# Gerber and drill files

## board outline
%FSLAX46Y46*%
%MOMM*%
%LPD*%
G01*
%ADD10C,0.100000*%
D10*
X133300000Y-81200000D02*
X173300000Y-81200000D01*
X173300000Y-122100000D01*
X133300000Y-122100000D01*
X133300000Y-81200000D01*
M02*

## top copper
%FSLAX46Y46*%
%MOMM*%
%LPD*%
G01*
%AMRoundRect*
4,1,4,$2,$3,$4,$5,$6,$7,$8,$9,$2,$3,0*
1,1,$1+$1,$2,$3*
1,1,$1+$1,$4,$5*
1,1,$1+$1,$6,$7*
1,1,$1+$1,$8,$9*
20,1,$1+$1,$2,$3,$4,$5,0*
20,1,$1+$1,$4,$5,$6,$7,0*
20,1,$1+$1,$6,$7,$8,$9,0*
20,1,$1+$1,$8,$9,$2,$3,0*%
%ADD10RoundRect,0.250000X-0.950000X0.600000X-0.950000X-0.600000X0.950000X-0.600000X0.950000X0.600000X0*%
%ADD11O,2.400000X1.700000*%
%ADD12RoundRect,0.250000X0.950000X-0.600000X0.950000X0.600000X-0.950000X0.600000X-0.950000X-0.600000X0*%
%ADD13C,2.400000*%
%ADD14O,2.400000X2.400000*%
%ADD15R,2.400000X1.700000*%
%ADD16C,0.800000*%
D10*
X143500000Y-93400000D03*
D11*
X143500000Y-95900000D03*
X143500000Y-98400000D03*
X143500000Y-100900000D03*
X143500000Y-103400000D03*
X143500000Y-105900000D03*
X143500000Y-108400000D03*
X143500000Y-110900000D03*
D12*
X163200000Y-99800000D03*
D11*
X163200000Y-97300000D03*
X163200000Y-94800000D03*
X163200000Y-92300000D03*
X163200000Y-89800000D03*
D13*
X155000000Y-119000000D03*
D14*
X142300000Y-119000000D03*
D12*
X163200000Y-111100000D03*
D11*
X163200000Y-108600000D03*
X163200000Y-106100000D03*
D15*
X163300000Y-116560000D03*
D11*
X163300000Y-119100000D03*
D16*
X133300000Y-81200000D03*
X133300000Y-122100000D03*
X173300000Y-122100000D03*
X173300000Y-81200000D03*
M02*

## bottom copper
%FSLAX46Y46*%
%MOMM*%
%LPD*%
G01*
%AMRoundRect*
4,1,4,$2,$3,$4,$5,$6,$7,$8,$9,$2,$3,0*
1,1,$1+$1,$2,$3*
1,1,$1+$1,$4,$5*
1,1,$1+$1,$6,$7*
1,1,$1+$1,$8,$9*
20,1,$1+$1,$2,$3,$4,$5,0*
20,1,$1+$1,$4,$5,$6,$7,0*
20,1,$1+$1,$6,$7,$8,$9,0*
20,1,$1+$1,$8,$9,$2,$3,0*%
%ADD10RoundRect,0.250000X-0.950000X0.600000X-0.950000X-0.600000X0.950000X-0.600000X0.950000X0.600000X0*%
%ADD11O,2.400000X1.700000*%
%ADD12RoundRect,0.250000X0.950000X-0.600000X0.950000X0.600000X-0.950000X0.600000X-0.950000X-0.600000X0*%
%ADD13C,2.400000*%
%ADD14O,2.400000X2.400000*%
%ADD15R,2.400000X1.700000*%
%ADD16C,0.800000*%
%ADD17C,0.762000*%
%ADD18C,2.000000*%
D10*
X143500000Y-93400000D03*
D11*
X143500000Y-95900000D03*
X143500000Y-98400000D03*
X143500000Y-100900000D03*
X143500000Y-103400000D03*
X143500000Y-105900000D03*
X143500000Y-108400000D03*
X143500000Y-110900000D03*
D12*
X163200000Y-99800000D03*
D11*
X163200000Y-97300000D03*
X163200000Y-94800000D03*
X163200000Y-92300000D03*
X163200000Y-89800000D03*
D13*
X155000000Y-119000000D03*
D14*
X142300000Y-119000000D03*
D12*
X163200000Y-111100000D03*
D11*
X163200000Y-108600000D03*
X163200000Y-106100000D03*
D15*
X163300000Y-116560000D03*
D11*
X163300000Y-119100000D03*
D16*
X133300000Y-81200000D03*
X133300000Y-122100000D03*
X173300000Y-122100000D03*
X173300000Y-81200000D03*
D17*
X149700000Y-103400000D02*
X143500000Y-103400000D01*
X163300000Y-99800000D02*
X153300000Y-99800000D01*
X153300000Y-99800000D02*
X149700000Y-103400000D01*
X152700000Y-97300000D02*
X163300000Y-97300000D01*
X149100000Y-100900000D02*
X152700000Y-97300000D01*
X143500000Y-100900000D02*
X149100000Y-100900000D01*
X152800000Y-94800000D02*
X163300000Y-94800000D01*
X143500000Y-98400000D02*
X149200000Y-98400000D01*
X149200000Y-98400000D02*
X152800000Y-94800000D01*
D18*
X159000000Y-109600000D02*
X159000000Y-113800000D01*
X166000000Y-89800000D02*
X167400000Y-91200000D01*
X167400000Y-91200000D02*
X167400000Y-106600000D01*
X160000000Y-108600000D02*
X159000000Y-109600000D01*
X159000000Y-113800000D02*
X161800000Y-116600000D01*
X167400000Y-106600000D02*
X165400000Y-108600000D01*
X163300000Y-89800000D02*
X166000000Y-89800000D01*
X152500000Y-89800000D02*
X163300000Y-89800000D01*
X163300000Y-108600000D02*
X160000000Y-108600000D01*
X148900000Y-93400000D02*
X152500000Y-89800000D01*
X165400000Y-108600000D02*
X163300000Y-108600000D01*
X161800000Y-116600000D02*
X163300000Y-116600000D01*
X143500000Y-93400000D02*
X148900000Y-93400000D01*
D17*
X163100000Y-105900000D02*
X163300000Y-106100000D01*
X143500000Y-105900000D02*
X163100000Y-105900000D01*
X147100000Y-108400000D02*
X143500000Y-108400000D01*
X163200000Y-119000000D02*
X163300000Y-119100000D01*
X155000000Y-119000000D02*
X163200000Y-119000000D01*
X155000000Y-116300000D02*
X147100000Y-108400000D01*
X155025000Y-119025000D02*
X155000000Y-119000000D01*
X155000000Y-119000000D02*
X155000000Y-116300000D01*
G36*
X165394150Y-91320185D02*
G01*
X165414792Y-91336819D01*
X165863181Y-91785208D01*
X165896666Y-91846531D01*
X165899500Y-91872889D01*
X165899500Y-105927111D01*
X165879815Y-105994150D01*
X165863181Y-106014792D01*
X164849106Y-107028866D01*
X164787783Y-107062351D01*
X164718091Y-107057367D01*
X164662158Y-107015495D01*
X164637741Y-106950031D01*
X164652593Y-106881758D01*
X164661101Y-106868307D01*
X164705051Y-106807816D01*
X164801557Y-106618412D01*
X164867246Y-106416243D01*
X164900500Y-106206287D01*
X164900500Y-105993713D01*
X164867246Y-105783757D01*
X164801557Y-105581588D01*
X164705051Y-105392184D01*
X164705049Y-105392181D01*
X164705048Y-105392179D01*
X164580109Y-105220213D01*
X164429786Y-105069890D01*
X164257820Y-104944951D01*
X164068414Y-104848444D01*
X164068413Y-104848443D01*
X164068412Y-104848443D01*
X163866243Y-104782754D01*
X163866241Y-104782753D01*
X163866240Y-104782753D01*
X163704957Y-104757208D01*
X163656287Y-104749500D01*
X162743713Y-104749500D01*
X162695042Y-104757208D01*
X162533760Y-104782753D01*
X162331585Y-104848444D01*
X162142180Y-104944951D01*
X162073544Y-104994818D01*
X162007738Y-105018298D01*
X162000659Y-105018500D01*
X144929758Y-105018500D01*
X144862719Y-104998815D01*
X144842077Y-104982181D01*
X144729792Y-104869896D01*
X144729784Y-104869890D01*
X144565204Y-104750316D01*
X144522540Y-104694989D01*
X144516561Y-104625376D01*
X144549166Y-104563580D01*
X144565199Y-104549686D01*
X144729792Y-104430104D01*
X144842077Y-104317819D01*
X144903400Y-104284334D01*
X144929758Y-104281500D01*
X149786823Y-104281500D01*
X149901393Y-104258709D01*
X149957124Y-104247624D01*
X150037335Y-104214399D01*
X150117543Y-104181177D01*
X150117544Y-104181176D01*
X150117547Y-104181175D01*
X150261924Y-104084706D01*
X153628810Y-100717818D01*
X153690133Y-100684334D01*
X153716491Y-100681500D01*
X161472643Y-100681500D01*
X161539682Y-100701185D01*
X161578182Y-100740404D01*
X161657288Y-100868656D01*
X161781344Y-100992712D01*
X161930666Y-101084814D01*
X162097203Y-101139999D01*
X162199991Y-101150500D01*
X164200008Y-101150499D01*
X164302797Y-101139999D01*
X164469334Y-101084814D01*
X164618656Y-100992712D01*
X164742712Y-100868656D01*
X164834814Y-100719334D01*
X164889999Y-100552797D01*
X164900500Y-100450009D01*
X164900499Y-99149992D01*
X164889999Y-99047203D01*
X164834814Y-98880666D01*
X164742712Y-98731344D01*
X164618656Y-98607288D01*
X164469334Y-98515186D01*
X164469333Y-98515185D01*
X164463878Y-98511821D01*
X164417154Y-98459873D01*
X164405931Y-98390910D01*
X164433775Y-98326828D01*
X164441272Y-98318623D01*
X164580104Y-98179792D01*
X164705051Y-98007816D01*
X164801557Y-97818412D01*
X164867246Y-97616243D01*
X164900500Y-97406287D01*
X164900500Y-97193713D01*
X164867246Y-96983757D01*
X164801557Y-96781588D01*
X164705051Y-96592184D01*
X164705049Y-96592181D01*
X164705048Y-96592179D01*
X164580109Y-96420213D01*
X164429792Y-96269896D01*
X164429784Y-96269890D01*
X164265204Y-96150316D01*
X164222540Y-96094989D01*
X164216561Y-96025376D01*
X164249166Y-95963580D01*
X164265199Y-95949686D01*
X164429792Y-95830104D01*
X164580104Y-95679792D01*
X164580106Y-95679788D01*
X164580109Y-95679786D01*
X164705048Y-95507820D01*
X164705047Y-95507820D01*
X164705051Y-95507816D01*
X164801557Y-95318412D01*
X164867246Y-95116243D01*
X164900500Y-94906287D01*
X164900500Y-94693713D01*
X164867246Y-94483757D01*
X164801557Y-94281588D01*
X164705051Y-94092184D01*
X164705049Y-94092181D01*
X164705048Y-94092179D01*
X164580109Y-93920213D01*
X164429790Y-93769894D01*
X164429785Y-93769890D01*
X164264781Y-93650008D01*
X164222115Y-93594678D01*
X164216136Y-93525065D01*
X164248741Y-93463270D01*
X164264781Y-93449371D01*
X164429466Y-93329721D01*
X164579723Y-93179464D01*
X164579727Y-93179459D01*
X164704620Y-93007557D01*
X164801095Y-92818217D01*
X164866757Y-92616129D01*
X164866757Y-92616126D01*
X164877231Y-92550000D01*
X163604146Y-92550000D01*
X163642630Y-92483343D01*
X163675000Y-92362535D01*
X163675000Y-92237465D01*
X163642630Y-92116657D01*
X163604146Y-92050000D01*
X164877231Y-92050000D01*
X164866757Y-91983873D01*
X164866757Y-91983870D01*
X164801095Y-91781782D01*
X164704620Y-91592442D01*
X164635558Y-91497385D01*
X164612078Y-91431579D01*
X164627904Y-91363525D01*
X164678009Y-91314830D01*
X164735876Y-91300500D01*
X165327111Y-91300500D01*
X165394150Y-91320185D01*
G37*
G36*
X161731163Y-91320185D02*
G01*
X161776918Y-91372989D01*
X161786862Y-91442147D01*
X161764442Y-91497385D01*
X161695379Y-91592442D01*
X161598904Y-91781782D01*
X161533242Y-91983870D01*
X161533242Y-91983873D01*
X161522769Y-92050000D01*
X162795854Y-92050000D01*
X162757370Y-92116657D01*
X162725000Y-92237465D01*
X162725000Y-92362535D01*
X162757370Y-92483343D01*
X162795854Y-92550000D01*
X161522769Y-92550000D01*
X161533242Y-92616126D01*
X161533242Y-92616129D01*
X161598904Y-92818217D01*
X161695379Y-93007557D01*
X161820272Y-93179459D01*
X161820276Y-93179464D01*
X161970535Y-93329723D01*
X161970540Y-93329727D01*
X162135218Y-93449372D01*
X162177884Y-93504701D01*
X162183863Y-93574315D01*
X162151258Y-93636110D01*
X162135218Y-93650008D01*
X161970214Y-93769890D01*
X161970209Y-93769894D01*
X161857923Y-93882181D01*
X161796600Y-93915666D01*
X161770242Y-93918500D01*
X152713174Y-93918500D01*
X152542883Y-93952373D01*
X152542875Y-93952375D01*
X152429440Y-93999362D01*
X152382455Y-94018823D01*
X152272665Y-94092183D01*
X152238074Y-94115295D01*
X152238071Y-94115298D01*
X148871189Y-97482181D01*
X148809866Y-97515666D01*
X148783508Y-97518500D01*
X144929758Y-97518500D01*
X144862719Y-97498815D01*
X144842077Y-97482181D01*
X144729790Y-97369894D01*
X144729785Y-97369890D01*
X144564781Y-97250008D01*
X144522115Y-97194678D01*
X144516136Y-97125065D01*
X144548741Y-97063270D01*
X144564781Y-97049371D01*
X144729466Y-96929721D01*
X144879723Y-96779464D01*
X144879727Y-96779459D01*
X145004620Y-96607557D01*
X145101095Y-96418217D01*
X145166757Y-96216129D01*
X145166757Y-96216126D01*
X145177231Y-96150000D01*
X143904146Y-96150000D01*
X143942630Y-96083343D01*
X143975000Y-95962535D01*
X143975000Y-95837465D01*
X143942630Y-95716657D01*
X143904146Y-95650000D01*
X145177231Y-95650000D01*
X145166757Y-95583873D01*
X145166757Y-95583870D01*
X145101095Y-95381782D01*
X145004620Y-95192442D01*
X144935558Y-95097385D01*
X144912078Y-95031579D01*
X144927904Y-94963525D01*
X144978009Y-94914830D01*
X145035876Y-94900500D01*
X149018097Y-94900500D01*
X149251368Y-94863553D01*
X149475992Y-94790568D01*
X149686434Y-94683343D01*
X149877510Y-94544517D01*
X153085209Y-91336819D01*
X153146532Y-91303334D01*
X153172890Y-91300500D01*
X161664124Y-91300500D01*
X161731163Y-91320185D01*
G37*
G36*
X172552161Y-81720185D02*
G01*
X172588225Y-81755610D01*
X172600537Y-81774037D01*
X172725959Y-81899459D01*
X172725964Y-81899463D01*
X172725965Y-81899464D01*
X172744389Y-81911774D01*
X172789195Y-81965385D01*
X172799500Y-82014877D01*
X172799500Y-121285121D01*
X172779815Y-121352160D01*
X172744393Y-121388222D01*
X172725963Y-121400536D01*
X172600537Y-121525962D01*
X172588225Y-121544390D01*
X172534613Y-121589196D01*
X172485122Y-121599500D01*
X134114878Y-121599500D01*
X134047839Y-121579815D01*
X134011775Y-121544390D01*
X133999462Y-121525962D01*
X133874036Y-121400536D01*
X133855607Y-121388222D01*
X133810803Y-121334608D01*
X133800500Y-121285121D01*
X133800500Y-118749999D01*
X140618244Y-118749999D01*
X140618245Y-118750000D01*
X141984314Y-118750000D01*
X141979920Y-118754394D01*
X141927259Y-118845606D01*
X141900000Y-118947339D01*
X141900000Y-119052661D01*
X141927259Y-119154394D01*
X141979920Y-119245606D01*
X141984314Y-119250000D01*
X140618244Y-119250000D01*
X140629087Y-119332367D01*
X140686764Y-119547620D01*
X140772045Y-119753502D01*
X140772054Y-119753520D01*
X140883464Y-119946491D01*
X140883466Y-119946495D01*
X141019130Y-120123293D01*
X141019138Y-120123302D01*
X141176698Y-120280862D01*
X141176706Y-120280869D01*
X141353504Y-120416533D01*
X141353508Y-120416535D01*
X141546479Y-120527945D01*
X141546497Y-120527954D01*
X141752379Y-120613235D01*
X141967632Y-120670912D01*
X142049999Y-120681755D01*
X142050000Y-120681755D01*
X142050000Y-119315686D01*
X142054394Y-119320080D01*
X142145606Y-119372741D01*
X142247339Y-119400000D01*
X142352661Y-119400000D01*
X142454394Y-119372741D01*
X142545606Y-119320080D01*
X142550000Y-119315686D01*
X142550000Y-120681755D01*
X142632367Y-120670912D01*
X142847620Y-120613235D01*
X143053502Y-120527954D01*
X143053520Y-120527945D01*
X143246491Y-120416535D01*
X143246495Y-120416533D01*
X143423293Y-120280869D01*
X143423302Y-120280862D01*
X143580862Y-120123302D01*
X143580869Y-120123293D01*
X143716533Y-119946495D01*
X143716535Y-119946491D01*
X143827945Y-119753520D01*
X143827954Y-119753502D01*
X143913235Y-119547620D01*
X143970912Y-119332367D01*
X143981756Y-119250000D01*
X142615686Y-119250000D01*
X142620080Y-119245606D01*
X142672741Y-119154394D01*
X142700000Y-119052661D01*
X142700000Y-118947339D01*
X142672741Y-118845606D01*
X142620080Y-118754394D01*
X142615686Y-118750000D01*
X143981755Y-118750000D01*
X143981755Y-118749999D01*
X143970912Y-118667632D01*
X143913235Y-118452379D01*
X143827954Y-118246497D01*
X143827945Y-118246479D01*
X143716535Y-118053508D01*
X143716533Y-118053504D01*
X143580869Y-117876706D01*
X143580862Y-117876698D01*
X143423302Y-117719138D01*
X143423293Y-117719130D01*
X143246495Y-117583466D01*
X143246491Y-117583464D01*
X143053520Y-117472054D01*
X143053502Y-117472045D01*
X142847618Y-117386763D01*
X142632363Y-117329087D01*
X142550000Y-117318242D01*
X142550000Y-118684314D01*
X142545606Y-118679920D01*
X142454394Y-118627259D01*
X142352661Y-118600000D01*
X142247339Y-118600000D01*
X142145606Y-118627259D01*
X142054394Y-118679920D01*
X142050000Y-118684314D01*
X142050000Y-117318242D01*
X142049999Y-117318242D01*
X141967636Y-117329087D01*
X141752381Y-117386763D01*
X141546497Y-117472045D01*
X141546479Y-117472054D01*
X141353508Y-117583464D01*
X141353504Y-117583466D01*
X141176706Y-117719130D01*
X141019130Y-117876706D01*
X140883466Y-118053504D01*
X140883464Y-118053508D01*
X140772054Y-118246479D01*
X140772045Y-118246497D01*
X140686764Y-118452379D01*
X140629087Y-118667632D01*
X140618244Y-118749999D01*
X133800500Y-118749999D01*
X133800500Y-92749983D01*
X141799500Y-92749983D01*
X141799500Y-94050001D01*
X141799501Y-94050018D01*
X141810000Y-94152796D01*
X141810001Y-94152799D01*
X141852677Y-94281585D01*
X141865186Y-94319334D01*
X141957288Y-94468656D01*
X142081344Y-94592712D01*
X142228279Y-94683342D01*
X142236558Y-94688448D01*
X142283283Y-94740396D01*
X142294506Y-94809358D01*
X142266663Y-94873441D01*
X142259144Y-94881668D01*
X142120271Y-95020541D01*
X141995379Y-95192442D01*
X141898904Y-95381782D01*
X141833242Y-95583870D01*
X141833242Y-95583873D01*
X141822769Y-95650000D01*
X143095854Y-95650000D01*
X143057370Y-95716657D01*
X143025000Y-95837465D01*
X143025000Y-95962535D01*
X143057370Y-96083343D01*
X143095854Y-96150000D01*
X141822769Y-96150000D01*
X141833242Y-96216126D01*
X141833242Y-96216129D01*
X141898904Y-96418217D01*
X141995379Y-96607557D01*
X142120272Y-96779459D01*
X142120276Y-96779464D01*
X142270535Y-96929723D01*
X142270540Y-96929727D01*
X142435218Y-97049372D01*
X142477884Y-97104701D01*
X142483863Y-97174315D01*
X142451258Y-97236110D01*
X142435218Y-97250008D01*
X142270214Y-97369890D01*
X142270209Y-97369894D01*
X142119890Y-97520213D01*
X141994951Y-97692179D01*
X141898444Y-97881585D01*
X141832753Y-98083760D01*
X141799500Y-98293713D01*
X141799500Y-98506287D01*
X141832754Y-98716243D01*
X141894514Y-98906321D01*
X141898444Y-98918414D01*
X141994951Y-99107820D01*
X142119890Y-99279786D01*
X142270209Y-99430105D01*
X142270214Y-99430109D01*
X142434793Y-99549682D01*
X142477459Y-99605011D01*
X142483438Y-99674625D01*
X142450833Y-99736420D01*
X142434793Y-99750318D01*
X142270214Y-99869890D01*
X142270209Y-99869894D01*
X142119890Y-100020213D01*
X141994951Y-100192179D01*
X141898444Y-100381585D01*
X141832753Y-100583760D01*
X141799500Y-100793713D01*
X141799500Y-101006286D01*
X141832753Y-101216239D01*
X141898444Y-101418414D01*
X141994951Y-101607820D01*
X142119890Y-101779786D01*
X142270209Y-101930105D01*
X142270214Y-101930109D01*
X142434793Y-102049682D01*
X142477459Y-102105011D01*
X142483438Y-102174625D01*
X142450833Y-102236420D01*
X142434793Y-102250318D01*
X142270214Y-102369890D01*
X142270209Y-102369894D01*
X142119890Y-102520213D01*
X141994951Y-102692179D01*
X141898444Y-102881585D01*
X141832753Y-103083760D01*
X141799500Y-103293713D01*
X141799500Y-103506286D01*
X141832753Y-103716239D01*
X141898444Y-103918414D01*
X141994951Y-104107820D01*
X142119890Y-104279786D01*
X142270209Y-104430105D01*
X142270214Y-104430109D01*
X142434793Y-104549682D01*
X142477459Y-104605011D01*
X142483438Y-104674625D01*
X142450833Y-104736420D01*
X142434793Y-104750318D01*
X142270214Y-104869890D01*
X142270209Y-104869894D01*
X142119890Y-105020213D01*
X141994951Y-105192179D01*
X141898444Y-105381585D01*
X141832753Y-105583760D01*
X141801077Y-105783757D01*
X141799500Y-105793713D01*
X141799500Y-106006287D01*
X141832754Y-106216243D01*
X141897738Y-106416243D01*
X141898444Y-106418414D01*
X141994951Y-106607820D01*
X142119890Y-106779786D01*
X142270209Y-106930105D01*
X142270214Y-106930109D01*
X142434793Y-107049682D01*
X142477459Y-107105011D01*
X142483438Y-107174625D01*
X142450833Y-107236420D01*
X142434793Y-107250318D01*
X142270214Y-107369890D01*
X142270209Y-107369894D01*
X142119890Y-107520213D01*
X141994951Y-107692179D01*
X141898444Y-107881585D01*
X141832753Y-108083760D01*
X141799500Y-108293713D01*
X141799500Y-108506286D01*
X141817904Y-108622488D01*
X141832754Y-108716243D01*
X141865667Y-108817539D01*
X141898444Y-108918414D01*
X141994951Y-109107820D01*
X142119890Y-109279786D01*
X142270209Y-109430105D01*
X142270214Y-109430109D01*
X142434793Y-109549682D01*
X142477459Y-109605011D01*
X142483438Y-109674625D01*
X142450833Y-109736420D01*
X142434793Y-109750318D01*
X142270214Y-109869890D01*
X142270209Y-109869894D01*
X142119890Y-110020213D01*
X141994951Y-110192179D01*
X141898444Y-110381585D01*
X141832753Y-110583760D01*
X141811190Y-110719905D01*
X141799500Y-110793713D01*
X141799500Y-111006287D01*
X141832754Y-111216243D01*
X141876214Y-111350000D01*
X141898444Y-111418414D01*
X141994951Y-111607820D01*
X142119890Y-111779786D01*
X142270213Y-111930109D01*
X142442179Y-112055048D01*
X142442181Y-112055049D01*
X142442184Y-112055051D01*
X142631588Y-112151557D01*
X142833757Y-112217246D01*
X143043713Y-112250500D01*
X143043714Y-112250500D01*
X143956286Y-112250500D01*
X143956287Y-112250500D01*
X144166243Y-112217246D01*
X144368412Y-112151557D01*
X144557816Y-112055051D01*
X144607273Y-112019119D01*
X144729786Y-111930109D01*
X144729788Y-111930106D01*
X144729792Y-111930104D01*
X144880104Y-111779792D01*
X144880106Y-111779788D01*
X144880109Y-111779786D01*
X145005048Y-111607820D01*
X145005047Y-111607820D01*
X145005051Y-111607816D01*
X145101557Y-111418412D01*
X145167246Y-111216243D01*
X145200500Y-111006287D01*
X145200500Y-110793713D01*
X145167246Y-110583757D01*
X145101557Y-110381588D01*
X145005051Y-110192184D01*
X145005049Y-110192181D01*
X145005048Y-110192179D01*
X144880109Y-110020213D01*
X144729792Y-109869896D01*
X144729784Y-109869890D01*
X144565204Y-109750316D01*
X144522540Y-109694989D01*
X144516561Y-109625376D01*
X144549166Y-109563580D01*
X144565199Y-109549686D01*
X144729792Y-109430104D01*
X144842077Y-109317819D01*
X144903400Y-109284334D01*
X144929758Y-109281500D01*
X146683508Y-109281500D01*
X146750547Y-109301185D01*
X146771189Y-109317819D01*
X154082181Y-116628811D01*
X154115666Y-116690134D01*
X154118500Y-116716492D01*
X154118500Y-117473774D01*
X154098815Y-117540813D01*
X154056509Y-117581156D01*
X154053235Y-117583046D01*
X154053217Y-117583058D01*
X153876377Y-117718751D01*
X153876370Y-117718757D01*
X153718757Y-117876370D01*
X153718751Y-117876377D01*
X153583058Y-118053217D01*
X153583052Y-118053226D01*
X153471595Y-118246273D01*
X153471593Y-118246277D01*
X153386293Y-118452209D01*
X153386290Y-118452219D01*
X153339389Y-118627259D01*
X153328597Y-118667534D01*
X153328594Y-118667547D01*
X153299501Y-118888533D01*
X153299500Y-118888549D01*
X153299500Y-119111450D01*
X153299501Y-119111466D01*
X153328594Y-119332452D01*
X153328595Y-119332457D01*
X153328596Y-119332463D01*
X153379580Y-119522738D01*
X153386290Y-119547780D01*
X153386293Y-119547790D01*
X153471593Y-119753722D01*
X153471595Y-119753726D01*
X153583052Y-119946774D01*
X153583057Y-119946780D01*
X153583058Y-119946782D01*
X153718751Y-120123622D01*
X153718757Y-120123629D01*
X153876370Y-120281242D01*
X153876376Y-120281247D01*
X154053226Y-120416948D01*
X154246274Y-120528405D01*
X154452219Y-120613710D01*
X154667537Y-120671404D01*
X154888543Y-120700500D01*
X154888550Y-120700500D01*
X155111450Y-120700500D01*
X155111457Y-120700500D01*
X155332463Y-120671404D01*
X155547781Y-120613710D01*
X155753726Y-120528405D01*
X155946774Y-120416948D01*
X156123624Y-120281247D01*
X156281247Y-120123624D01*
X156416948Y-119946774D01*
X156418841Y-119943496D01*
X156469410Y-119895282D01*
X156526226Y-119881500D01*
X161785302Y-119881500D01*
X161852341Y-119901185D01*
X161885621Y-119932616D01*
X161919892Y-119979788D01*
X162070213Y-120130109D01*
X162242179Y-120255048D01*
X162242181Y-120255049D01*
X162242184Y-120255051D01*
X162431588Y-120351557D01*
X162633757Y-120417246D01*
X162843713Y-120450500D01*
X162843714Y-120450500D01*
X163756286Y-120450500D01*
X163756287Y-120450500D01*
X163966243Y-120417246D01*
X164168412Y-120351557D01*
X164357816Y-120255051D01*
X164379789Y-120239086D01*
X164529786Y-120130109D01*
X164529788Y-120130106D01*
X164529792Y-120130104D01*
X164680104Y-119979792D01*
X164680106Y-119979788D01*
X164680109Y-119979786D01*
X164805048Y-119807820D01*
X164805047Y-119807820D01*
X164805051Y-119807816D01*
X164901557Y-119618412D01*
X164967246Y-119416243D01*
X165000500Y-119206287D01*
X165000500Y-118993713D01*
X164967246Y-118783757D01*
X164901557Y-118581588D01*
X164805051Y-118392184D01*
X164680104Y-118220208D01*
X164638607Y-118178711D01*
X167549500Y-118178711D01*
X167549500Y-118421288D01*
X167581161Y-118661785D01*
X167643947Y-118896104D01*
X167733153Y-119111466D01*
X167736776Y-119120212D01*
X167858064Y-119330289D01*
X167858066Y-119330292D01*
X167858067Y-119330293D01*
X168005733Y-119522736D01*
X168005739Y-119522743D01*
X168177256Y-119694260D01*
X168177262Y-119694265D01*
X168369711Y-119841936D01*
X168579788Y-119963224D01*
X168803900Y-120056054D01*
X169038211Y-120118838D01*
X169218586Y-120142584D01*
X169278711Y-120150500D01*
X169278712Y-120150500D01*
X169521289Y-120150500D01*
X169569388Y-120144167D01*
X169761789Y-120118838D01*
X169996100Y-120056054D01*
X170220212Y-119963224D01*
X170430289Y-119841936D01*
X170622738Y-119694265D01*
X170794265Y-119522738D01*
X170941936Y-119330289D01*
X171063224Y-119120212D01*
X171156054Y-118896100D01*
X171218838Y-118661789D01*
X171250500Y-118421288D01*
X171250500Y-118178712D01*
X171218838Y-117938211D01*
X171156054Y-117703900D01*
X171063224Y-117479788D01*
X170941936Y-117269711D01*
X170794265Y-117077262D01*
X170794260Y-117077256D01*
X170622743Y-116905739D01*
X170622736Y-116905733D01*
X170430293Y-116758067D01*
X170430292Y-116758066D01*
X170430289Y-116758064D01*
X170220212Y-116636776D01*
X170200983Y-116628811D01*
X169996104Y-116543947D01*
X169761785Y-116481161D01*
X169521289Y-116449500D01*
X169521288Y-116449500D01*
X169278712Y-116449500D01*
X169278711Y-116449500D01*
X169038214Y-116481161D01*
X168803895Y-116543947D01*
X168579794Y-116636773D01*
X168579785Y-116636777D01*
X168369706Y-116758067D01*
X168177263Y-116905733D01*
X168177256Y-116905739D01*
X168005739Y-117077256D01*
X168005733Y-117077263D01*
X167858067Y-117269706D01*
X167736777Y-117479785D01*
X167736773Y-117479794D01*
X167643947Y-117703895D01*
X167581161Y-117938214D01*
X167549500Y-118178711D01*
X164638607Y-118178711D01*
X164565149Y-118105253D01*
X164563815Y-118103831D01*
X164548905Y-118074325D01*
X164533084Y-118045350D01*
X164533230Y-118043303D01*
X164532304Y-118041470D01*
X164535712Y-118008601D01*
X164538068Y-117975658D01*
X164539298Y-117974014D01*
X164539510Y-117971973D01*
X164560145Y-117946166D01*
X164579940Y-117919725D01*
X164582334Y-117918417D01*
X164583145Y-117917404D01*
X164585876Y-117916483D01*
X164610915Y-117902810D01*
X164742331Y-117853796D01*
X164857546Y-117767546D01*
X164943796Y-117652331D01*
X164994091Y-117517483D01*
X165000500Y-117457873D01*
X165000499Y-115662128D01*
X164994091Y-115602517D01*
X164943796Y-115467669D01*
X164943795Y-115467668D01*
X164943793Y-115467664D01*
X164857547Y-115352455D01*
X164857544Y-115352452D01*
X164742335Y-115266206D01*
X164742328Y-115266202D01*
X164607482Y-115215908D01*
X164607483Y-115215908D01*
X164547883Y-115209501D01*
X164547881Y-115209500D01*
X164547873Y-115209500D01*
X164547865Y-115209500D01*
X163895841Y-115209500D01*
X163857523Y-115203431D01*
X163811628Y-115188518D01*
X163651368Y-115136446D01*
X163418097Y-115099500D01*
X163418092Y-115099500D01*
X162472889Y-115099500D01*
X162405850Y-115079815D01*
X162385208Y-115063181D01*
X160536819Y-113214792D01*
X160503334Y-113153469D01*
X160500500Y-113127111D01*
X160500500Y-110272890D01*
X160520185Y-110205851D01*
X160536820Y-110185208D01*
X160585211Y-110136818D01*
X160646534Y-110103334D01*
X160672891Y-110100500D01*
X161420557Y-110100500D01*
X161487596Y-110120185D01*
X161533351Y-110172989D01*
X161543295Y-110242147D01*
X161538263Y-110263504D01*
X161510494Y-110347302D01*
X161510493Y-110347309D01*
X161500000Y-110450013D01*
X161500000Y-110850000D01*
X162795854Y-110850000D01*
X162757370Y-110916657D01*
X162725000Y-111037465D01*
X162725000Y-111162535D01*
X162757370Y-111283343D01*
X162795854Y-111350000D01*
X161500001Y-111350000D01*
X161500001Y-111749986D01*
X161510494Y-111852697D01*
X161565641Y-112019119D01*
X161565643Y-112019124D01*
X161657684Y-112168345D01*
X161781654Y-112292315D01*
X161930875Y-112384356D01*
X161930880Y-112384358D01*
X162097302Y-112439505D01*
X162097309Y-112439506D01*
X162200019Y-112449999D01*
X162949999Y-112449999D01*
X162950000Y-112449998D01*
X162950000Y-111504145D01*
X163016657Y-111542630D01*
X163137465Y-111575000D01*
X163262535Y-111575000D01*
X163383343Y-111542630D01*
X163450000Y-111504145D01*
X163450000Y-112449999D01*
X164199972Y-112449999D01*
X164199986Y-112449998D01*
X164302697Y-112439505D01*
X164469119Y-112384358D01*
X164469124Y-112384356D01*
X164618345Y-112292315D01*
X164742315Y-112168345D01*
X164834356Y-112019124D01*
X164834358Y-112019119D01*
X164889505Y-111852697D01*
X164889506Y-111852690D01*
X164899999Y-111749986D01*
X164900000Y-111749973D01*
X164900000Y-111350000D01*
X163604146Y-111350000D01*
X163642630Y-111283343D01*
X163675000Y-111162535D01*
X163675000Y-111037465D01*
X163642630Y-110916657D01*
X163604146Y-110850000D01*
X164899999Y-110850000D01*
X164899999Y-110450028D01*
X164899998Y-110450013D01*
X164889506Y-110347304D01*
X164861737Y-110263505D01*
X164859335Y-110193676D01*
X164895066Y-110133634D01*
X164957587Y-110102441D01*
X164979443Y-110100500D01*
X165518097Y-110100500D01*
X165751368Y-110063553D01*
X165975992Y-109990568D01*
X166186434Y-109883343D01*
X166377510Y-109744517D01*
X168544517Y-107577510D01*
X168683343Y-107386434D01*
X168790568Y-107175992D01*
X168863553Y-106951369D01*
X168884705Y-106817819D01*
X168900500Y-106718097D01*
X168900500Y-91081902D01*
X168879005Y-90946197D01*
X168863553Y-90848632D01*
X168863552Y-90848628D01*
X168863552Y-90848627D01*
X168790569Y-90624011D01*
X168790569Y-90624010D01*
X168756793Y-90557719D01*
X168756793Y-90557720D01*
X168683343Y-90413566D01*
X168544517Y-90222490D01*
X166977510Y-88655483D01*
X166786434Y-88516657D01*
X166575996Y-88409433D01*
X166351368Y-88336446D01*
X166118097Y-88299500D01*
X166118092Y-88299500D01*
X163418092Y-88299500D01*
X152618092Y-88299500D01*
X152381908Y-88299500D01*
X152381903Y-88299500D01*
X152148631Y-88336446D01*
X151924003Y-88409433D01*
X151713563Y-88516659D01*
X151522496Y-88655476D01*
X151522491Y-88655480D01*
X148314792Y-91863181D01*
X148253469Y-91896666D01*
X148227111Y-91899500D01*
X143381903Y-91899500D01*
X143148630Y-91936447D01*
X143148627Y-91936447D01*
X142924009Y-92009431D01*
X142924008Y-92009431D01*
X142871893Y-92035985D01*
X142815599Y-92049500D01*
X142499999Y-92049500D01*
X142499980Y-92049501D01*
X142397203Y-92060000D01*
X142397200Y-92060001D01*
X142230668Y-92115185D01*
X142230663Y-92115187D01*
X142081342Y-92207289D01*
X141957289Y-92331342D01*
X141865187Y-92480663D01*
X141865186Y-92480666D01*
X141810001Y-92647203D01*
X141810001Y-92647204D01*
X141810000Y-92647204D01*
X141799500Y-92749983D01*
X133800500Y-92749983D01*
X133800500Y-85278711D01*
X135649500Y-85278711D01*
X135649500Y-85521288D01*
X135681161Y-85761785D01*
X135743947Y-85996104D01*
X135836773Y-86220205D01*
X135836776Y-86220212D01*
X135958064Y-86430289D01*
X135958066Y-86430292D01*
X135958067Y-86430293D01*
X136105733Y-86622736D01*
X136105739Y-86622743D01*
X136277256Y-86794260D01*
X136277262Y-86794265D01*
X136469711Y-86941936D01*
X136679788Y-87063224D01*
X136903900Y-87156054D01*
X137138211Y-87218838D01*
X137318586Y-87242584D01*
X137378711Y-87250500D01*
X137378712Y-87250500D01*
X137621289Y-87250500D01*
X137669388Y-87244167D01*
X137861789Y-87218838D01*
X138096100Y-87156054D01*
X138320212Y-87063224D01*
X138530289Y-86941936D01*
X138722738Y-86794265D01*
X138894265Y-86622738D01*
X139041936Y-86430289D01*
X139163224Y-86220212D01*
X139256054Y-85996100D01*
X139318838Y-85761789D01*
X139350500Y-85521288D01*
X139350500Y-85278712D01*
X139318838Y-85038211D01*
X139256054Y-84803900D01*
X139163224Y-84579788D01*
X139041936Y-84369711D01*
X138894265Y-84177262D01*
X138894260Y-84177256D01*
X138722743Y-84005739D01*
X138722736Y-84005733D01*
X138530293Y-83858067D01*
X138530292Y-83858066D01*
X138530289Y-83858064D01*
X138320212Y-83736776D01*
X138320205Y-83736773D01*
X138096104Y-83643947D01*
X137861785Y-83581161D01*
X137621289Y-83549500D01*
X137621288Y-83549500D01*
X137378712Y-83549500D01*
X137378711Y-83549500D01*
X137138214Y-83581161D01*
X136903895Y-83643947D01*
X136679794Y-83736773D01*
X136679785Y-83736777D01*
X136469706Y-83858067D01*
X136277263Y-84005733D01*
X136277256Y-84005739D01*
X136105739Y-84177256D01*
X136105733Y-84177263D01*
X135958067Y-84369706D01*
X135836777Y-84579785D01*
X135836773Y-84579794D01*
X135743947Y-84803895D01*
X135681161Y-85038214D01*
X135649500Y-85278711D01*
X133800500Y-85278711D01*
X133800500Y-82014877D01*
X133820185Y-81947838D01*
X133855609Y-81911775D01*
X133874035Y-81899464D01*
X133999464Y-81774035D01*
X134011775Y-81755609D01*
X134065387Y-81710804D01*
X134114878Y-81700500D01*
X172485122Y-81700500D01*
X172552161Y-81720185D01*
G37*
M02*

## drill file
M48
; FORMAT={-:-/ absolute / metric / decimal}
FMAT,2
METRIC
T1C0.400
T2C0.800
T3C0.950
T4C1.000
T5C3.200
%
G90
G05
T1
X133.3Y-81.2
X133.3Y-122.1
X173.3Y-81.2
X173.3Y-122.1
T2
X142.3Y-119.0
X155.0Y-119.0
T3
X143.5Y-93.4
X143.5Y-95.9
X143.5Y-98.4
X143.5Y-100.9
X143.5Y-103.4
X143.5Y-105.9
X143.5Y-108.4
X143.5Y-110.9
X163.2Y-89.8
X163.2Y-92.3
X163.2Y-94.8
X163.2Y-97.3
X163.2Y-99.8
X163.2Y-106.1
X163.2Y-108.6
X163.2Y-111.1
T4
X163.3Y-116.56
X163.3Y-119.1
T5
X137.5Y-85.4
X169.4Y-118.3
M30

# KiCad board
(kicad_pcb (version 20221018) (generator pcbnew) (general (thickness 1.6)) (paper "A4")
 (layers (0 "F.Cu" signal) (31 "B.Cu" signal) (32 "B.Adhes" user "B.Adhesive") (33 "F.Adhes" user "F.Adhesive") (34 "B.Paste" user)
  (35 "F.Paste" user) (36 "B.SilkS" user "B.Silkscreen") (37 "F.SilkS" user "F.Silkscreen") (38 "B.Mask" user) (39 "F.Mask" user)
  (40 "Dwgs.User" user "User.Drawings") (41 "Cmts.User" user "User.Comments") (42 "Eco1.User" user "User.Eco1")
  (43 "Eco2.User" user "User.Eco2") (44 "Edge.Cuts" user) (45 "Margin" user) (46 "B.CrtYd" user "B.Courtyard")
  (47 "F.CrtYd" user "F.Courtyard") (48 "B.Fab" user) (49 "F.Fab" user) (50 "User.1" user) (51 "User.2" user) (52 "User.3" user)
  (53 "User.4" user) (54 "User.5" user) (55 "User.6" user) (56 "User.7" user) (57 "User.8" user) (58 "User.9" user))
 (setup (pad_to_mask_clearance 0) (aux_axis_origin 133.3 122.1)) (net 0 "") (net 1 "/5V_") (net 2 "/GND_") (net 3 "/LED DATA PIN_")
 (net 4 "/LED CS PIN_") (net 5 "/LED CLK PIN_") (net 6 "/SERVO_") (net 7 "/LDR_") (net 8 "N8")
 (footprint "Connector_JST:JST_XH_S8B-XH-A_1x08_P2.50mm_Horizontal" (layer "F.Cu") (at 143.5 93.4 -90)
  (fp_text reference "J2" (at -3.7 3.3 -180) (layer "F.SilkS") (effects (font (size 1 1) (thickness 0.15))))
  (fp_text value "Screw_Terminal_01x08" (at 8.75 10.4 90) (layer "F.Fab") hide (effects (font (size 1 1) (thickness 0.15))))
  (pad "1" thru_hole roundrect (at 0 0 270) (size 1.7 2.4) (drill 0.95) (layers "*.Cu" "*.Mask") (roundrect_rratio 0.147059) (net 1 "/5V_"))
  (pad "2" thru_hole oval (at 2.5 0 270) (size 1.7 2.4) (drill 0.95) (layers "*.Cu" "*.Mask") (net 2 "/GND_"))
  (pad "3" thru_hole oval (at 5 0 270) (size 1.7 2.4) (drill 0.95) (layers "*.Cu" "*.Mask") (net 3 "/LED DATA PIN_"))
  (pad "4" thru_hole oval (at 7.5 0 270) (size 1.7 2.4) (drill 0.95) (layers "*.Cu" "*.Mask") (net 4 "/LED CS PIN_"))
  (pad "5" thru_hole oval (at 10 0 270) (size 1.7 2.4) (drill 0.95) (layers "*.Cu" "*.Mask") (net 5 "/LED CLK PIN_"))
  (pad "6" thru_hole oval (at 12.5 0 270) (size 1.7 2.4) (drill 0.95) (layers "*.Cu" "*.Mask") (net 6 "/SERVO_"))
  (pad "7" thru_hole oval (at 15 0 270) (size 1.7 2.4) (drill 0.95) (layers "*.Cu" "*.Mask") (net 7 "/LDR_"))
  (pad "8" thru_hole oval (at 17.5 0 270) (size 1.7 2.4) (drill 0.95) (layers "*.Cu" "*.Mask") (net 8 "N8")))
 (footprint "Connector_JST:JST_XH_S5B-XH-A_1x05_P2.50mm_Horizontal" (layer "F.Cu") (at 163.2 99.8 90)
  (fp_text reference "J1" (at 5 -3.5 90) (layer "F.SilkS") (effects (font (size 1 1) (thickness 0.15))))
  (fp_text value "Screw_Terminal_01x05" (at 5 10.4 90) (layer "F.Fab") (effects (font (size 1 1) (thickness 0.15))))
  (pad "1" thru_hole roundrect (at 0 0 90) (size 1.7 2.4) (drill 0.95) (layers "*.Cu" "*.Mask") (roundrect_rratio 0.147059)
   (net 5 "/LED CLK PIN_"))
  (pad "2" thru_hole oval (at 2.5 0 90) (size 1.7 2.4) (drill 0.95) (layers "*.Cu" "*.Mask") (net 4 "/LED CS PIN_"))
  (pad "3" thru_hole oval (at 5 0 90) (size 1.7 2.4) (drill 0.95) (layers "*.Cu" "*.Mask") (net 3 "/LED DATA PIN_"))
  (pad "4" thru_hole oval (at 7.5 0 90) (size 1.7 2.4) (drill 0.95) (layers "*.Cu" "*.Mask") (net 2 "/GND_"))
  (pad "5" thru_hole oval (at 10 0 90) (size 1.7 2.4) (drill 0.95) (layers "*.Cu" "*.Mask") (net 1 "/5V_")))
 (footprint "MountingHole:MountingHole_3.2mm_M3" (layer "F.Cu") (at 137.5 85.4)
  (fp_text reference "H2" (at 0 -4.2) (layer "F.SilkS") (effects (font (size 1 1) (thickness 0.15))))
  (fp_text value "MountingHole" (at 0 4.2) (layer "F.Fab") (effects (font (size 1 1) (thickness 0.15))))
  (pad "" np_thru_hole circle (at 0 0) (size 3.2 3.2) (drill 3.2) (layers "*.Cu" "*.Mask")))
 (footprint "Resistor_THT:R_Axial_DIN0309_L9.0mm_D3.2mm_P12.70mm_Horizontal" (layer "F.Cu") (at 155 119 180)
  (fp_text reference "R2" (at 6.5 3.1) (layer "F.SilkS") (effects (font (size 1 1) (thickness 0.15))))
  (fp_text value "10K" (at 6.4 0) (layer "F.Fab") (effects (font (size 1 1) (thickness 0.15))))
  (pad "1" thru_hole circle (at 0 0 180) (size 2.4 2.4) (drill 0.8) (layers "*.Cu" "*.Mask") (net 7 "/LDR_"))
  (pad "2" thru_hole oval (at 12.7 0 180) (size 2.4 2.4) (drill 0.8) (layers "*.Cu" "*.Mask") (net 2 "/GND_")))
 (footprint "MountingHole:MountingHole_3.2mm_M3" (layer "F.Cu") (at 169.4 118.3)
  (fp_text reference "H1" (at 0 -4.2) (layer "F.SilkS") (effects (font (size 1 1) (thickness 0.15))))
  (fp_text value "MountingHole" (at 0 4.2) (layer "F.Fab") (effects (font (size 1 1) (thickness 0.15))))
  (pad "" np_thru_hole circle (at 0 0) (size 3.2 3.2) (drill 3.2) (layers "*.Cu" "*.Mask")))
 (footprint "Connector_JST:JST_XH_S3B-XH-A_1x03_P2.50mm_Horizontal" (layer "F.Cu") (at 163.2 111.1 90)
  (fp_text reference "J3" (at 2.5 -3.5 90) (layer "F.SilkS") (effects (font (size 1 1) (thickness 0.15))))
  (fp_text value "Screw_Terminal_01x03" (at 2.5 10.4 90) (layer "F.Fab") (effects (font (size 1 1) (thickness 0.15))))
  (pad "1" thru_hole roundrect (at 0 0 90) (size 1.7 2.4) (drill 0.95) (layers "*.Cu" "*.Mask") (roundrect_rratio 0.147059) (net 2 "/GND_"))
  (pad "2" thru_hole oval (at 2.5 0 90) (size 1.7 2.4) (drill 0.95) (layers "*.Cu" "*.Mask") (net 1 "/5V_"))
  (pad "3" thru_hole oval (at 5 0 90) (size 1.7 2.4) (drill 0.95) (layers "*.Cu" "*.Mask") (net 6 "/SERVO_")))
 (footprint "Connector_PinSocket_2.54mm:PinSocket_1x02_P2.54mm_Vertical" (layer "F.Cu") (at 163.3 116.56)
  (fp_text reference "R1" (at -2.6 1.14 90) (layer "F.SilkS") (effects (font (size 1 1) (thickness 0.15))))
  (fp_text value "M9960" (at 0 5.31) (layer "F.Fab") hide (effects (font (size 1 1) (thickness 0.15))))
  (pad "1" thru_hole rect (at 0 0) (size 2.4 1.7) (drill 1) (layers "*.Cu" "*.Mask") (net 1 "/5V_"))
  (pad "2" thru_hole oval (at 0 2.54) (size 2.4 1.7) (drill 1) (layers "*.Cu" "*.Mask") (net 7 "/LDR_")))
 (gr_rect (start 133.3 81.2) (end 173.3 122.1) (stroke (width 0.1) (type default)) (fill none) (layer "Edge.Cuts"))
 (via (at 133.3 81.2) (size 0.8) (drill 0.4) (layers "F.Cu" "B.Cu") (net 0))
 (via (at 133.3 122.1) (size 0.8) (drill 0.4) (layers "F.Cu" "B.Cu") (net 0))
 (via (at 173.3 122.1) (size 0.8) (drill 0.4) (layers "F.Cu" "B.Cu") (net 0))
 (via (at 173.3 81.2) (size 0.8) (drill 0.4) (layers "F.Cu" "B.Cu") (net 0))
 (segment (start 149.7 103.4) (end 143.5 103.4) (width 0.762) (layer "B.Cu") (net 5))
 (segment (start 163.3 99.8) (end 153.3 99.8) (width 0.762) (layer "B.Cu") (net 5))
 (segment (start 153.3 99.8) (end 149.7 103.4) (width 0.762) (layer "B.Cu") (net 5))
 (segment (start 152.7 97.3) (end 163.3 97.3) (width 0.762) (layer "B.Cu") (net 4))
 (segment (start 149.1 100.9) (end 152.7 97.3) (width 0.762) (layer "B.Cu") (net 4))
 (segment (start 143.5 100.9) (end 149.1 100.9) (width 0.762) (layer "B.Cu") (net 4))
 (segment (start 152.8 94.8) (end 163.3 94.8) (width 0.762) (layer "B.Cu") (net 3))
 (segment (start 143.5 98.4) (end 149.2 98.4) (width 0.762) (layer "B.Cu") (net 3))
 (segment (start 149.2 98.4) (end 152.8 94.8) (width 0.762) (layer "B.Cu") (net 3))
 (segment (start 159 109.6) (end 159 113.8) (width 2) (layer "B.Cu") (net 1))
 (segment (start 166 89.8) (end 167.4 91.2) (width 2) (layer "B.Cu") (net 1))
 (segment (start 167.4 91.2) (end 167.4 106.6) (width 2) (layer "B.Cu") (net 1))
 (segment (start 160 108.6) (end 159 109.6) (width 2) (layer "B.Cu") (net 1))
 (segment (start 159 113.8) (end 161.8 116.6) (width 2) (layer "B.Cu") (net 1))
 (segment (start 167.4 106.6) (end 165.4 108.6) (width 2) (layer "B.Cu") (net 1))
 (segment (start 163.3 89.8) (end 166 89.8) (width 2) (layer "B.Cu") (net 1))
 (segment (start 152.5 89.8) (end 163.3 89.8) (width 2) (layer "B.Cu") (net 1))
 (segment (start 163.3 108.6) (end 160 108.6) (width 2) (layer "B.Cu") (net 1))
 (segment (start 148.9 93.4) (end 152.5 89.8) (width 2) (layer "B.Cu") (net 1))
 (segment (start 165.4 108.6) (end 163.3 108.6) (width 2) (layer "B.Cu") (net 1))
 (segment (start 161.8 116.6) (end 163.3 116.6) (width 2) (layer "B.Cu") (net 1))
 (segment (start 143.5 93.4) (end 148.9 93.4) (width 2) (layer "B.Cu") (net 1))
 (segment (start 163.1 105.9) (end 163.3 106.1) (width 0.762) (layer "B.Cu") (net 6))
 (segment (start 143.5 105.9) (end 163.1 105.9) (width 0.762) (layer "B.Cu") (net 6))
 (segment (start 147.1 108.4) (end 143.5 108.4) (width 0.762) (layer "B.Cu") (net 7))
 (segment (start 163.2 119) (end 163.3 119.1) (width 0.762) (layer "B.Cu") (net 7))
 (segment (start 155 119) (end 163.2 119) (width 0.762) (layer "B.Cu") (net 7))
 (segment (start 155 116.3) (end 147.1 108.4) (width 0.762) (layer "B.Cu") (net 7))
 (segment (start 155.025 119.025) (end 155 119) (width 0.762) (layer "B.Cu") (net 7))
 (segment (start 155 119) (end 155 116.3) (width 0.762) (layer "B.Cu") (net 7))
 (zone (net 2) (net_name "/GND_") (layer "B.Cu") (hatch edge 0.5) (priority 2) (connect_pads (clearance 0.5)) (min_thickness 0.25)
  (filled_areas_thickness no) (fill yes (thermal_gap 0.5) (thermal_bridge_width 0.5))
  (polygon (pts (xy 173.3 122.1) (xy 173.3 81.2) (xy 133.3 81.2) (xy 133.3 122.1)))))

